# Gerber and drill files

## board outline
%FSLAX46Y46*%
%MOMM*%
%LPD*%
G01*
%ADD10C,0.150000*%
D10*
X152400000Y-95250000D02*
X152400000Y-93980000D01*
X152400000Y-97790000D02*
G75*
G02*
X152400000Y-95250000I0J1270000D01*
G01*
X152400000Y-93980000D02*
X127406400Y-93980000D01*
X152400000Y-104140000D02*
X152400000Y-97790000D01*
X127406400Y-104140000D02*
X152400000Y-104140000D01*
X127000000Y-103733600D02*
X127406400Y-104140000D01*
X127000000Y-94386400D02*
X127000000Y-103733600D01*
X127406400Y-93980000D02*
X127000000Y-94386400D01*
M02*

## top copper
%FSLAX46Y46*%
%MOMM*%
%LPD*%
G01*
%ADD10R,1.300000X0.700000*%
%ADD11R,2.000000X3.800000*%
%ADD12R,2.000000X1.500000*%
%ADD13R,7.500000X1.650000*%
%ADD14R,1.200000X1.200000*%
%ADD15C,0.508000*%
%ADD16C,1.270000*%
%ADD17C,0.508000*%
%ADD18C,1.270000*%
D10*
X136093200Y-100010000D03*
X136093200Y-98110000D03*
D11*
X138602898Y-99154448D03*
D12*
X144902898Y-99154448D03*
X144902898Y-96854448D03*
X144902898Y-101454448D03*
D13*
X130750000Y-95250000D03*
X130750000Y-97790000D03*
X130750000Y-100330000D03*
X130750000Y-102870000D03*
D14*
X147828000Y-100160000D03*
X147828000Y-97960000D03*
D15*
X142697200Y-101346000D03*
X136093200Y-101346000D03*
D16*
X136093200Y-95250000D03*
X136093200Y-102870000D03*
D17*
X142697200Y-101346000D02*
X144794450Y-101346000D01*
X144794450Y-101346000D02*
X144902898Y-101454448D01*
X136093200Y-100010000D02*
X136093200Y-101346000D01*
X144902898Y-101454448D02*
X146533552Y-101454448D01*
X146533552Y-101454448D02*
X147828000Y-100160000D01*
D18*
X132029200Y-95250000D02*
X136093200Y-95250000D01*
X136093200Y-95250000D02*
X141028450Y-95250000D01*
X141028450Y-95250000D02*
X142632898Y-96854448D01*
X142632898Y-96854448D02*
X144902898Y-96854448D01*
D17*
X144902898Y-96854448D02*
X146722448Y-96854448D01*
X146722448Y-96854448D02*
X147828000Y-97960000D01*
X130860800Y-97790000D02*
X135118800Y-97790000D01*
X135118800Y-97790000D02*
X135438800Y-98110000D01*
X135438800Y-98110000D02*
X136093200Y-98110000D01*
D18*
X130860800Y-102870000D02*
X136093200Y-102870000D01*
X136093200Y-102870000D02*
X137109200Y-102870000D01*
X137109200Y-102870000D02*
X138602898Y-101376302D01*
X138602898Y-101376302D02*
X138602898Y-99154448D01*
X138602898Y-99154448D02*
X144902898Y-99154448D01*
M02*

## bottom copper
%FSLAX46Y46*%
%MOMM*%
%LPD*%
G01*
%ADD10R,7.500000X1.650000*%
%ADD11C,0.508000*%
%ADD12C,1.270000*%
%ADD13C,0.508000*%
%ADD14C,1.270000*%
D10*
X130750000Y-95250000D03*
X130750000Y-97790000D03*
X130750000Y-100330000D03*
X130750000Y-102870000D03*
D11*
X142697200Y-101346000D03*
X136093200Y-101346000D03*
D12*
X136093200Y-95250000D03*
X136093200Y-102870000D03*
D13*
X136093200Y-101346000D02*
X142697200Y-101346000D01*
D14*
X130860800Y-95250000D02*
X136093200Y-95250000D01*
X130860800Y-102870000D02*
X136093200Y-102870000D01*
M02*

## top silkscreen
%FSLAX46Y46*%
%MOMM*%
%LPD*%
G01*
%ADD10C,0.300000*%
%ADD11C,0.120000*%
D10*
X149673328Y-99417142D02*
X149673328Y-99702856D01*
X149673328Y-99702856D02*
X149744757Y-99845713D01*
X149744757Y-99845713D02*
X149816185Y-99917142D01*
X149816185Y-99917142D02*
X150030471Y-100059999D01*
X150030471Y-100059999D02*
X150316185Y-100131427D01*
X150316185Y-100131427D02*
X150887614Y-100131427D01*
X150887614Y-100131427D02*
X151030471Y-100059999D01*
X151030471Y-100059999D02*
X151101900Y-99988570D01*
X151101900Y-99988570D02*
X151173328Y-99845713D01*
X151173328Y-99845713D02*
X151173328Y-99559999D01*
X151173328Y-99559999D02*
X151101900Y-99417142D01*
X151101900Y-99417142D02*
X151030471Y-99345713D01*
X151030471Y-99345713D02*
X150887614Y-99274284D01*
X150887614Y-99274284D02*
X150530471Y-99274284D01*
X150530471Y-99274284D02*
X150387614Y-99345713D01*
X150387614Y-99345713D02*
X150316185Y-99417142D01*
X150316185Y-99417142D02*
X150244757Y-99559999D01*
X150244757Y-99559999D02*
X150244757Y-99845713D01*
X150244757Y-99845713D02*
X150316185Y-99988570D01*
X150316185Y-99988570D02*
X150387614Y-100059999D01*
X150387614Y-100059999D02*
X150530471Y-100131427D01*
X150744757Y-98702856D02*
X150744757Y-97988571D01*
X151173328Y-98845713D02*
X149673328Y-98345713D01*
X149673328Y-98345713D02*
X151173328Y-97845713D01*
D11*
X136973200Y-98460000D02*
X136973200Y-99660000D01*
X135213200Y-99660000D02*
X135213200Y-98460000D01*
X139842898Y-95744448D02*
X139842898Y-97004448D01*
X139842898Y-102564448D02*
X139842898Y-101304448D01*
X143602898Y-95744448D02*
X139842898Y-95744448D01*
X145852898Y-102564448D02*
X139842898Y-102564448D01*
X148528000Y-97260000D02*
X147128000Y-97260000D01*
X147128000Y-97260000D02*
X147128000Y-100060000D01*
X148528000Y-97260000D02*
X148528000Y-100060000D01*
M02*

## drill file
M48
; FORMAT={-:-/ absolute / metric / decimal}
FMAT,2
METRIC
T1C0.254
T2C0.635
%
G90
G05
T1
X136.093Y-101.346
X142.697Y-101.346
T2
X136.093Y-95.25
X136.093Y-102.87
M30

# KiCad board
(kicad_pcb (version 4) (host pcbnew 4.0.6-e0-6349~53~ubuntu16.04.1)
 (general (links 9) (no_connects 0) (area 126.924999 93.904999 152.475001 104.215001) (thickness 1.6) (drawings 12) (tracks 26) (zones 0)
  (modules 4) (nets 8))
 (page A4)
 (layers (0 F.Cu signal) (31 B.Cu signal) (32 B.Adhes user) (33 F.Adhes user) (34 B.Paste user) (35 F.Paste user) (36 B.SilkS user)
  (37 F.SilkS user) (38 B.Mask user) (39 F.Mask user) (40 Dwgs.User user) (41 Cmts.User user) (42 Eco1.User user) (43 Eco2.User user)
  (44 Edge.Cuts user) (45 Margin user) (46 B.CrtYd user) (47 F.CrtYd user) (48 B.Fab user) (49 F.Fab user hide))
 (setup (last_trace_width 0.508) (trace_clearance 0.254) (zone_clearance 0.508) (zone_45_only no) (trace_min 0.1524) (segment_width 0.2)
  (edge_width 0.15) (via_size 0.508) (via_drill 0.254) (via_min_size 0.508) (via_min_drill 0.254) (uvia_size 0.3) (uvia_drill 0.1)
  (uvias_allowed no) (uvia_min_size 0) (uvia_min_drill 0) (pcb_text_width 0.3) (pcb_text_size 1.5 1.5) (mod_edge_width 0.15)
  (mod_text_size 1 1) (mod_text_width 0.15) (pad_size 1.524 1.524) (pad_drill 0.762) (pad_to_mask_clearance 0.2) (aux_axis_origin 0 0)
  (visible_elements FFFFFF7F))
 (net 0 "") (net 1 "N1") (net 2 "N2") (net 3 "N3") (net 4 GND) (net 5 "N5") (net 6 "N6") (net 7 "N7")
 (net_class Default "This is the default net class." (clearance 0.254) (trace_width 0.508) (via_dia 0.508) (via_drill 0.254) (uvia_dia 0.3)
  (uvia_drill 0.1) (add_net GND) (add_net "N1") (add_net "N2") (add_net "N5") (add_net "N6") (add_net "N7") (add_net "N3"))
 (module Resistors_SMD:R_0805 (layer F.Cu) (at 136.0932 99.06 90)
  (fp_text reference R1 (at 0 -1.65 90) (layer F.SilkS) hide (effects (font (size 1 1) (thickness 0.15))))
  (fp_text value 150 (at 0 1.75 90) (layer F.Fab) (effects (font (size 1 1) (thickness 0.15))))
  (fp_line (start 0.6 0.88) (end -0.6 0.88) (layer F.SilkS) (width 0.12))
  (fp_line (start -0.6 -0.88) (end 0.6 -0.88) (layer F.SilkS) (width 0.12))
  (pad 1 smd rect (at -0.95 0 90) (size 0.7 1.3) (layers F.Cu F.Paste F.Mask) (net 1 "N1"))
  (pad 2 smd rect (at 0.95 0 90) (size 0.7 1.3) (layers F.Cu F.Paste F.Mask) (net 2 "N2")))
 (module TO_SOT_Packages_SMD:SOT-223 (layer F.Cu) (at 141.752898 99.154448 180)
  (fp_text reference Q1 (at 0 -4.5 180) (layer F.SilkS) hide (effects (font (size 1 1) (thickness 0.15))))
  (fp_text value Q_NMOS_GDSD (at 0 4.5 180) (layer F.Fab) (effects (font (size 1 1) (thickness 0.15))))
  (fp_line (start 1.91 3.41) (end 1.91 2.15) (layer F.SilkS) (width 0.12))
  (fp_line (start 1.91 -3.41) (end 1.91 -2.15) (layer F.SilkS) (width 0.12))
  (fp_line (start -1.85 3.41) (end 1.91 3.41) (layer F.SilkS) (width 0.12))
  (fp_line (start -4.1 -3.41) (end 1.91 -3.41) (layer F.SilkS) (width 0.12))
  (pad 4 smd rect (at 3.15 0 180) (size 2 3.8) (layers F.Cu F.Paste F.Mask) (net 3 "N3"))
  (pad 2 smd rect (at -3.15 0 180) (size 2 1.5) (layers F.Cu F.Paste F.Mask) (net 3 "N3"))
  (pad 3 smd rect (at -3.15 2.3 180) (size 2 1.5) (layers F.Cu F.Paste F.Mask) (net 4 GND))
  (pad 1 smd rect (at -3.15 -2.3 180) (size 2 1.5) (layers F.Cu F.Paste F.Mask) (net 1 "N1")))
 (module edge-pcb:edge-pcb (layer F.Cu) (at 127 99.06 270)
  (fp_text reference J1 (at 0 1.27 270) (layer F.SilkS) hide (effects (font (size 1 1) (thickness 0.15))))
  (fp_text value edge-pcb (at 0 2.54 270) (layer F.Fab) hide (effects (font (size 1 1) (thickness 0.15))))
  (pad 1 smd rect (at -3.81 -3.75 270) (size 1.65 7.5) (layers F.Cu F.Paste F.Mask) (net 4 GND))
  (pad 2 smd rect (at -3.81 -3.75 270) (size 1.65 7.5) (layers B.Cu B.Paste B.Mask) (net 4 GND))
  (pad 3 smd rect (at -1.27 -3.75 270) (size 1.65 7.5) (layers F.Cu F.Paste F.Mask) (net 2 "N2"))
  (pad 4 smd rect (at -1.27 -3.75 270) (size 1.65 7.5) (layers B.Cu B.Paste B.Mask) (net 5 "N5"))
  (pad 5 smd rect (at 1.27 -3.75 270) (size 1.65 7.5) (layers F.Cu F.Paste F.Mask) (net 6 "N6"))
  (pad 6 smd rect (at 1.27 -3.75 270) (size 1.65 7.5) (layers B.Cu B.Paste B.Mask) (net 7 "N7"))
  (pad 7 smd rect (at 3.81 -3.75 270) (size 1.65 7.5) (layers F.Cu F.Paste F.Mask) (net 3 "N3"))
  (pad 8 smd rect (at 3.81 -3.75 270) (size 1.65 7.5) (layers B.Cu B.Paste B.Mask) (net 3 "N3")))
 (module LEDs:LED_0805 (layer F.Cu) (at 147.828 99.06 270)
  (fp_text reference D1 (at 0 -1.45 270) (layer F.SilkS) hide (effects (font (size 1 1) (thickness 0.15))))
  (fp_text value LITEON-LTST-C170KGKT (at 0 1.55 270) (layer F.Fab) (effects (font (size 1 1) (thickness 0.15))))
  (fp_line (start -1.8 -0.7) (end -1.8 0.7) (layer F.SilkS) (width 0.12))
  (fp_line (start -1.8 0.7) (end 1 0.7) (layer F.SilkS) (width 0.12))
  (fp_line (start -1.8 -0.7) (end 1 -0.7) (layer F.SilkS) (width 0.12))
  (pad 2 smd rect (at 1.1 0 90) (size 1.2 1.2) (layers F.Cu F.Paste F.Mask) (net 1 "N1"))
  (pad 1 smd rect (at -1.1 0 90) (size 1.2 1.2) (layers F.Cu F.Paste F.Mask) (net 4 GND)))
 (gr_line (start 152.4 95.25) (end 152.4 93.98) (layer Edge.Cuts) (width 0.15))
 (gr_arc (start 152.4 96.52) (end 152.4 97.79) (angle 180) (layer Edge.Cuts) (width 0.15))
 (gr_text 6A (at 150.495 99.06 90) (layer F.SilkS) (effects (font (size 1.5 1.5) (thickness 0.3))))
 (gr_line (start 152.4 93.98) (end 127.4064 93.98) (layer Edge.Cuts) (width 0.15))
 (gr_line (start 152.4 104.14) (end 152.4 97.79) (layer Edge.Cuts) (width 0.15))
 (gr_line (start 127.4064 104.14) (end 152.4 104.14) (layer Edge.Cuts) (width 0.15))
 (gr_line (start 127 103.7336) (end 127.4064 104.14) (layer Edge.Cuts) (width 0.15))
 (gr_line (start 127 94.3864) (end 127 103.7336) (layer Edge.Cuts) (width 0.15))
 (gr_line (start 127.4064 93.98) (end 127 94.3864) (layer Edge.Cuts) (width 0.15))
 (segment (start 142.6972 101.346) (end 144.79445 101.346) (width 0.508) (layer F.Cu) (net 1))
 (segment (start 144.79445 101.346) (end 144.902898 101.454448) (width 0.508) (layer F.Cu) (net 1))
 (segment (start 136.0932 101.346) (end 142.6972 101.346) (width 0.508) (layer B.Cu) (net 1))
 (via (at 142.6972 101.346) (size 0.508) (drill 0.254) (layers F.Cu B.Cu) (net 1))
 (segment (start 136.0932 100.01) (end 136.0932 101.346) (width 0.508) (layer F.Cu) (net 1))
 (via (at 136.0932 101.346) (size 0.508) (drill 0.254) (layers F.Cu B.Cu) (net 1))
 (segment (start 144.902898 101.454448) (end 146.533552 101.454448) (width 0.508) (layer F.Cu) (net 1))
 (segment (start 146.533552 101.454448) (end 147.828 100.16) (width 0.508) (layer F.Cu) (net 1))
 (segment (start 132.0292 95.25) (end 136.0932 95.25) (width 1.27) (layer F.Cu) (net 4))
 (segment (start 136.0932 95.25) (end 141.02845 95.25) (width 1.27) (layer F.Cu) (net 4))
 (segment (start 130.8608 95.25) (end 136.0932 95.25) (width 1.27) (layer B.Cu) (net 4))
 (via (at 136.0932 95.25) (size 1.27) (drill 0.635) (layers F.Cu B.Cu) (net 4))
 (segment (start 141.02845 95.25) (end 142.632898 96.854448) (width 1.27) (layer F.Cu) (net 4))
 (segment (start 142.632898 96.854448) (end 144.902898 96.854448) (width 1.27) (layer F.Cu) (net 4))
 (segment (start 144.902898 96.854448) (end 146.722448 96.854448) (width 0.508) (layer F.Cu) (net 4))
 (segment (start 146.722448 96.854448) (end 147.828 97.96) (width 0.508) (layer F.Cu) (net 4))
 (segment (start 130.8608 97.79) (end 135.1188 97.79) (width 0.508) (layer F.Cu) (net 2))
 (segment (start 135.1188 97.79) (end 135.4388 98.11) (width 0.508) (layer F.Cu) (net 2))
 (segment (start 135.4388 98.11) (end 136.0932 98.11) (width 0.508) (layer F.Cu) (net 2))
 (segment (start 130.8608 102.87) (end 136.0932 102.87) (width 1.27) (layer F.Cu) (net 3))
 (segment (start 136.0932 102.87) (end 137.1092 102.87) (width 1.27) (layer F.Cu) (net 3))
 (via (at 136.0932 102.87) (size 1.27) (drill 0.635) (layers F.Cu B.Cu) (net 3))
 (segment (start 130.8608 102.87) (end 136.0932 102.87) (width 1.27) (layer B.Cu) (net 3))
 (segment (start 137.1092 102.87) (end 138.602898 101.376302) (width 1.27) (layer F.Cu) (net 3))
 (segment (start 138.602898 101.376302) (end 138.602898 99.154448) (width 1.27) (layer F.Cu) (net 3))
 (segment (start 138.602898 99.154448) (end 144.902898 99.154448) (width 1.27) (layer F.Cu) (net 3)))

